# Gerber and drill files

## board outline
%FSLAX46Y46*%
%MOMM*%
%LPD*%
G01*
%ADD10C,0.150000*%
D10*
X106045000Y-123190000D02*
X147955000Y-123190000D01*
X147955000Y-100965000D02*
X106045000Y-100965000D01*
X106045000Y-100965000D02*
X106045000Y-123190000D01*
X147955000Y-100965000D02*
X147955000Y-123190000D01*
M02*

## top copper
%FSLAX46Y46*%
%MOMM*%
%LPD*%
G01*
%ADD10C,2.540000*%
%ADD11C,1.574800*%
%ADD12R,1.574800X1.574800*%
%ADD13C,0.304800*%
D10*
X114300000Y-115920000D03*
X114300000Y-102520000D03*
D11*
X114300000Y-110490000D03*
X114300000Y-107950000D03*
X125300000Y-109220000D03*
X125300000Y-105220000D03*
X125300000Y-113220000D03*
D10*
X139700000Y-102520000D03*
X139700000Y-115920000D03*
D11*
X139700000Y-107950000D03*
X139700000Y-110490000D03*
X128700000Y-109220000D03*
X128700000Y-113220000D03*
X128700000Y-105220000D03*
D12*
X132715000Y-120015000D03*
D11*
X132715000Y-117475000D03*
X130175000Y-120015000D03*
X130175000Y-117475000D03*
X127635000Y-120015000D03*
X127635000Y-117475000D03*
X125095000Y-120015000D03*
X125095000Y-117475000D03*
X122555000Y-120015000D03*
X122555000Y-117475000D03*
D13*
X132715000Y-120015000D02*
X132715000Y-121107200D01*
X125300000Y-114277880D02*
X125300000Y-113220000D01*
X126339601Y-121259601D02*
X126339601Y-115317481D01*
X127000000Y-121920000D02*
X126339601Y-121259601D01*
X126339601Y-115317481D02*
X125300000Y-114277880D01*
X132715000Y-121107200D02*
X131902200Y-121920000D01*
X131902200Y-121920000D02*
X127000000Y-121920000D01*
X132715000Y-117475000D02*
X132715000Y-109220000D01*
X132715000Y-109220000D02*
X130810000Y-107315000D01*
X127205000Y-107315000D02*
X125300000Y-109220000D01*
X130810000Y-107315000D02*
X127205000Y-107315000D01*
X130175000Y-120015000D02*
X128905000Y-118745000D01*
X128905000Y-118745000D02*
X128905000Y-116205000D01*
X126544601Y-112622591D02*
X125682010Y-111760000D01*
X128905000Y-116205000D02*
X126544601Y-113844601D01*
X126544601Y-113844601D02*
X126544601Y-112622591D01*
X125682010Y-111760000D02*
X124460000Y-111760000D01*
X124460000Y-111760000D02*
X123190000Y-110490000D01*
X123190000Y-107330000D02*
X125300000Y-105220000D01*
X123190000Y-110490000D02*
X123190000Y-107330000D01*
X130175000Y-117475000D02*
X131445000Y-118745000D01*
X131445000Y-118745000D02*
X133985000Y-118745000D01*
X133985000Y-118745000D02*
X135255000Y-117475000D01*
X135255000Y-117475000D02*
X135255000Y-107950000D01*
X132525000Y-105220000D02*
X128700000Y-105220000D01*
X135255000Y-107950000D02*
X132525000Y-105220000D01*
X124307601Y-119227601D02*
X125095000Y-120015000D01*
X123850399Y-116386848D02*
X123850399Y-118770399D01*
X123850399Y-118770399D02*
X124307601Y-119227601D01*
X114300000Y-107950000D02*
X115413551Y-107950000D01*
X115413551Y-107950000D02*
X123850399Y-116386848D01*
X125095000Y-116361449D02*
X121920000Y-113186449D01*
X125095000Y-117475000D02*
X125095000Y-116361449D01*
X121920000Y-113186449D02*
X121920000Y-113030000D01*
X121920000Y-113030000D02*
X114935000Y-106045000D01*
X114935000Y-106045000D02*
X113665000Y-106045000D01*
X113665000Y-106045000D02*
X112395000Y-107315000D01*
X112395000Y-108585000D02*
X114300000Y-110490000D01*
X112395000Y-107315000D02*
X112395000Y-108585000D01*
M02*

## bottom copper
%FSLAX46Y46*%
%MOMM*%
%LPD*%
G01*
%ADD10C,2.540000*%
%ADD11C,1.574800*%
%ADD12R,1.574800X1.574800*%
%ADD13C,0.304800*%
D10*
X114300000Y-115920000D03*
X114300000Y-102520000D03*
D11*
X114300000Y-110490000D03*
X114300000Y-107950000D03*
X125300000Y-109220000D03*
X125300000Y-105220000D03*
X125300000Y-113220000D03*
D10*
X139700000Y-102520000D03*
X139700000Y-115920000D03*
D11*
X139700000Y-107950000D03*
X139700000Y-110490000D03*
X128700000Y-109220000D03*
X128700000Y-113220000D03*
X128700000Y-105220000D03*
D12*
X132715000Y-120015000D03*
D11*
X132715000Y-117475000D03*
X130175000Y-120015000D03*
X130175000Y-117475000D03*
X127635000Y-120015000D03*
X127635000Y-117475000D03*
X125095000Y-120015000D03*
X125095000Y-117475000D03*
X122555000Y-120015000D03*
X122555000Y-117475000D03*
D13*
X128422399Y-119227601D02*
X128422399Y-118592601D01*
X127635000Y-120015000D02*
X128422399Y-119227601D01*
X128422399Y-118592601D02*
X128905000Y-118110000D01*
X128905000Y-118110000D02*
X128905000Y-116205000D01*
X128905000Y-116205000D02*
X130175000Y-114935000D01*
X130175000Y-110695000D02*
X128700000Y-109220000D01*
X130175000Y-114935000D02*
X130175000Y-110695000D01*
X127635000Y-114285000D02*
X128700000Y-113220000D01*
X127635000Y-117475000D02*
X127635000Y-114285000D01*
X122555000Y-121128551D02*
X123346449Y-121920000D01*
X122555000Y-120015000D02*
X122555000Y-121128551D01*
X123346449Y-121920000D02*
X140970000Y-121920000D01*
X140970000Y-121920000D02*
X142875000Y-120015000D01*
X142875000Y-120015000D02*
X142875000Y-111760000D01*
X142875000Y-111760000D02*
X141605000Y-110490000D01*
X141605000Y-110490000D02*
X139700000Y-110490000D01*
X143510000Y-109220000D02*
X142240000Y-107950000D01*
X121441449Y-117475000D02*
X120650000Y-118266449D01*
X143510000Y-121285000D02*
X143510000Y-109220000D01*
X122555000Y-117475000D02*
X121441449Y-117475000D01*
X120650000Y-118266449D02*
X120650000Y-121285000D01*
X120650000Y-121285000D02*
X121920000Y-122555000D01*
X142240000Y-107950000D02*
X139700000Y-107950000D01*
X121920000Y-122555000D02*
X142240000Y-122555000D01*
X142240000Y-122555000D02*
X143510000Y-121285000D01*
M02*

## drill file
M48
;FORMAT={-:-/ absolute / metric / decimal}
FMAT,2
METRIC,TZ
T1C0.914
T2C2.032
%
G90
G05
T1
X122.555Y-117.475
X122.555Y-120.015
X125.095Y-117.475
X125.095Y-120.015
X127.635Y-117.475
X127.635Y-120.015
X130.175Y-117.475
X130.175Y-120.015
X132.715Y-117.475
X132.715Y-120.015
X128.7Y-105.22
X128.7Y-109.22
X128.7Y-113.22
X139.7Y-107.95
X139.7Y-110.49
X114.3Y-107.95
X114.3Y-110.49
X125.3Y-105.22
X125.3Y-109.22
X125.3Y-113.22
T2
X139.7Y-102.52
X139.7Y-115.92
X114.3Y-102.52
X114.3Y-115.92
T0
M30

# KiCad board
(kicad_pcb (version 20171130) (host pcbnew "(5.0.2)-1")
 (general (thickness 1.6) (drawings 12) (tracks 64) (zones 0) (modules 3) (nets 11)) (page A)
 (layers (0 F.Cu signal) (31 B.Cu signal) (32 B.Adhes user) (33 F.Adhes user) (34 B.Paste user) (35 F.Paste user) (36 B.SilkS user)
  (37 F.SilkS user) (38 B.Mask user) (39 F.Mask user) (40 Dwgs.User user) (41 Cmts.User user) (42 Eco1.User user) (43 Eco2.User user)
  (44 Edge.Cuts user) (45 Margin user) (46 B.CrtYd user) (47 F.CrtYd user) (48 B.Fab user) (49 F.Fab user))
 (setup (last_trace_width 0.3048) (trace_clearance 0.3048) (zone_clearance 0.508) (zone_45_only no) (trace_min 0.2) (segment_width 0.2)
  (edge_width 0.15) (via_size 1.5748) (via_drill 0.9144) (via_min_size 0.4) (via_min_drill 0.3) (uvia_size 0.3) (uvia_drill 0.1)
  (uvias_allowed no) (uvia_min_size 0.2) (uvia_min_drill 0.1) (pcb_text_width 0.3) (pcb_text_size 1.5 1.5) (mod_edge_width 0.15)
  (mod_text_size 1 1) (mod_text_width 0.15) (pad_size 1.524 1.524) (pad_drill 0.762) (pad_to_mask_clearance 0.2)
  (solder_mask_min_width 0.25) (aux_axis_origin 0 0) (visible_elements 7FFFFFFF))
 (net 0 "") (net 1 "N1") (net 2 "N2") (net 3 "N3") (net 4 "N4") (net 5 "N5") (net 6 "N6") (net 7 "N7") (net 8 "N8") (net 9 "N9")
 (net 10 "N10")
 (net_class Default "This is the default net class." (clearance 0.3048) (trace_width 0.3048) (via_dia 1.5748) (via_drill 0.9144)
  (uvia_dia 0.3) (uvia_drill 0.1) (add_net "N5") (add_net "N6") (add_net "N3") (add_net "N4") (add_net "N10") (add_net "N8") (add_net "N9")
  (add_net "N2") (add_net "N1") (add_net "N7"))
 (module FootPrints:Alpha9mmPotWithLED (layer F.Cu) (at 114.3 109.22 90)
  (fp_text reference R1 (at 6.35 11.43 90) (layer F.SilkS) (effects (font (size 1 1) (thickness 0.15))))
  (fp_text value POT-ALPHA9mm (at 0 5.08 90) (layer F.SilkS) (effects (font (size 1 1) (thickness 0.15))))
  (pad "" thru_hole circle (at -6.7 0 90) (size 2.54 2.54) (drill 2.032) (layers *.Cu *.Mask F.SilkS))
  (pad "" thru_hole circle (at 6.7 0 90) (size 2.54 2.54) (drill 2.032) (layers *.Cu *.Mask F.SilkS))
  (pad 4 thru_hole circle (at -1.27 0 90) (size 1.5748 1.5748) (drill 0.9144) (layers *.Cu *.Mask F.SilkS) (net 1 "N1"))
  (pad 5 thru_hole circle (at 1.27 0 90) (size 1.5748 1.5748) (drill 0.9144) (layers *.Cu *.Mask F.SilkS) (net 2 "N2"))
  (pad 2 thru_hole circle (at 0 11 90) (size 1.5748 1.5748) (drill 0.9144) (layers *.Cu *.Mask F.SilkS) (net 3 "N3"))
  (pad 3 thru_hole circle (at 4 11 90) (size 1.5748 1.5748) (drill 0.9144) (layers *.Cu *.Mask F.SilkS) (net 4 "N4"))
  (pad 1 thru_hole circle (at -4 11 90) (size 1.5748 1.5748) (drill 0.9144) (layers *.Cu *.Mask F.SilkS) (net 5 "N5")))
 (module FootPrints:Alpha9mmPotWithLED (layer F.Cu) (at 139.7 109.22 270)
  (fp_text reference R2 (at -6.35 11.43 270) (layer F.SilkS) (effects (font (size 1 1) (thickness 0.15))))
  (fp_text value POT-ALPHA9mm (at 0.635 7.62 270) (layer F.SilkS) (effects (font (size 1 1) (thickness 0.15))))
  (pad "" thru_hole circle (at -6.7 0 270) (size 2.54 2.54) (drill 2.032) (layers *.Cu *.Mask F.SilkS))
  (pad "" thru_hole circle (at 6.7 0 270) (size 2.54 2.54) (drill 2.032) (layers *.Cu *.Mask F.SilkS))
  (pad 4 thru_hole circle (at -1.27 0 270) (size 1.5748 1.5748) (drill 0.9144) (layers *.Cu *.Mask F.SilkS) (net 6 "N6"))
  (pad 5 thru_hole circle (at 1.27 0 270) (size 1.5748 1.5748) (drill 0.9144) (layers *.Cu *.Mask F.SilkS) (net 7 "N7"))
  (pad 2 thru_hole circle (at 0 11 270) (size 1.5748 1.5748) (drill 0.9144) (layers *.Cu *.Mask F.SilkS) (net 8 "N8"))
  (pad 3 thru_hole circle (at 4 11 270) (size 1.5748 1.5748) (drill 0.9144) (layers *.Cu *.Mask F.SilkS) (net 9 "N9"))
  (pad 1 thru_hole circle (at -4 11 270) (size 1.5748 1.5748) (drill 0.9144) (layers *.Cu *.Mask F.SilkS) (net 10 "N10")))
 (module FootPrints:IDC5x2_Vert (layer B.Cu) (at 127.635 118.745)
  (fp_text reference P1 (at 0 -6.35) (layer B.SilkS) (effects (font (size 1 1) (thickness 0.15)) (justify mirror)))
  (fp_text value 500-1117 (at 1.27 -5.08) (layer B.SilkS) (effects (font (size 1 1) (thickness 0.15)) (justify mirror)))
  (pad 1 thru_hole rect (at 5.08 1.27) (size 1.5748 1.5748) (drill 0.9144) (layers *.Cu *.Mask B.SilkS) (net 5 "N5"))
  (pad 2 thru_hole circle (at 5.08 -1.27) (size 1.5748 1.5748) (drill 0.9144) (layers *.Cu *.Mask B.SilkS) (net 3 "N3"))
  (pad 3 thru_hole circle (at 2.54 1.27) (size 1.5748 1.5748) (drill 0.9144) (layers *.Cu *.Mask B.SilkS) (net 4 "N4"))
  (pad 4 thru_hole circle (at 2.54 -1.27) (size 1.5748 1.5748) (drill 0.9144) (layers *.Cu *.Mask B.SilkS) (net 10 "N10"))
  (pad 5 thru_hole circle (at 0 1.27) (size 1.5748 1.5748) (drill 0.9144) (layers *.Cu *.Mask B.SilkS) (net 8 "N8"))
  (pad 6 thru_hole circle (at 0 -1.27) (size 1.5748 1.5748) (drill 0.9144) (layers *.Cu *.Mask B.SilkS) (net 9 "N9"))
  (pad 7 thru_hole circle (at -2.54 1.27) (size 1.5748 1.5748) (drill 0.9144) (layers *.Cu *.Mask B.SilkS) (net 2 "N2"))
  (pad 8 thru_hole circle (at -2.54 -1.27) (size 1.5748 1.5748) (drill 0.9144) (layers *.Cu *.Mask B.SilkS) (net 1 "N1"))
  (pad 9 thru_hole circle (at -5.08 1.27) (size 1.5748 1.5748) (drill 0.9144) (layers *.Cu *.Mask B.SilkS) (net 7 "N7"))
  (pad 10 thru_hole circle (at -5.08 -1.27) (size 1.5748 1.5748) (drill 0.9144) (layers *.Cu *.Mask B.SilkS) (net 6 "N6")))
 (gr_line (start 106.045 123.19) (end 147.955 123.19) (layer Edge.Cuts) (width 0.15))
 (gr_line (start 147.955 100.965) (end 106.045 100.965) (layer Edge.Cuts) (width 0.15))
 (gr_line (start 106.045 100.965) (end 106.045 123.19) (layer Edge.Cuts) (width 0.15))
 (gr_line (start 147.955 100.965) (end 147.955 123.19) (layer Edge.Cuts) (width 0.15))
 (segment (start 132.715 120.015) (end 132.715 121.1072) (width 0.3048) (layer F.Cu) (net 5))
 (segment (start 125.3 114.27788) (end 125.3 113.22) (width 0.3048) (layer F.Cu) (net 5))
 (segment (start 126.339601 121.259601) (end 126.339601 115.317481) (width 0.3048) (layer F.Cu) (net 5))
 (segment (start 127 121.92) (end 126.339601 121.259601) (width 0.3048) (layer F.Cu) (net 5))
 (segment (start 126.339601 115.317481) (end 125.3 114.27788) (width 0.3048) (layer F.Cu) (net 5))
 (segment (start 132.715 121.1072) (end 131.9022 121.92) (width 0.3048) (layer F.Cu) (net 5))
 (segment (start 131.9022 121.92) (end 127 121.92) (width 0.3048) (layer F.Cu) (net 5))
 (segment (start 132.715 117.475) (end 132.715 109.22) (width 0.3048) (layer F.Cu) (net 3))
 (segment (start 132.715 109.22) (end 130.81 107.315) (width 0.3048) (layer F.Cu) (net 3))
 (segment (start 127.205 107.315) (end 125.3 109.22) (width 0.3048) (layer F.Cu) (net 3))
 (segment (start 130.81 107.315) (end 127.205 107.315) (width 0.3048) (layer F.Cu) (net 3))
 (segment (start 130.175 120.015) (end 128.905 118.745) (width 0.3048) (layer F.Cu) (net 4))
 (segment (start 128.905 118.745) (end 128.905 116.205) (width 0.3048) (layer F.Cu) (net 4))
 (segment (start 126.544601 112.622591) (end 125.68201 111.76) (width 0.3048) (layer F.Cu) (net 4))
 (segment (start 128.905 116.205) (end 126.544601 113.844601) (width 0.3048) (layer F.Cu) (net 4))
 (segment (start 126.544601 113.844601) (end 126.544601 112.622591) (width 0.3048) (layer F.Cu) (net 4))
 (segment (start 125.68201 111.76) (end 124.46 111.76) (width 0.3048) (layer F.Cu) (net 4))
 (segment (start 124.46 111.76) (end 123.19 110.49) (width 0.3048) (layer F.Cu) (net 4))
 (segment (start 123.19 107.33) (end 125.3 105.22) (width 0.3048) (layer F.Cu) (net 4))
 (segment (start 123.19 110.49) (end 123.19 107.33) (width 0.3048) (layer F.Cu) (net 4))
 (segment (start 130.175 117.475) (end 131.445 118.745) (width 0.3048) (layer F.Cu) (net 10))
 (segment (start 131.445 118.745) (end 133.985 118.745) (width 0.3048) (layer F.Cu) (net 10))
 (segment (start 133.985 118.745) (end 135.255 117.475) (width 0.3048) (layer F.Cu) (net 10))
 (segment (start 135.255 117.475) (end 135.255 107.95) (width 0.3048) (layer F.Cu) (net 10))
 (segment (start 132.525 105.22) (end 128.7 105.22) (width 0.3048) (layer F.Cu) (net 10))
 (segment (start 135.255 107.95) (end 132.525 105.22) (width 0.3048) (layer F.Cu) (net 10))
 (segment (start 128.422399 119.227601) (end 128.422399 118.592601) (width 0.3048) (layer B.Cu) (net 8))
 (segment (start 127.635 120.015) (end 128.422399 119.227601) (width 0.3048) (layer B.Cu) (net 8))
 (segment (start 128.422399 118.592601) (end 128.905 118.11) (width 0.3048) (layer B.Cu) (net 8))
 (segment (start 128.905 118.11) (end 128.905 116.205) (width 0.3048) (layer B.Cu) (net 8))
 (segment (start 128.905 116.205) (end 130.175 114.935) (width 0.3048) (layer B.Cu) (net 8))
 (segment (start 130.175 110.695) (end 128.7 109.22) (width 0.3048) (layer B.Cu) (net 8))
 (segment (start 130.175 114.935) (end 130.175 110.695) (width 0.3048) (layer B.Cu) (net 8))
 (segment (start 127.635 114.285) (end 128.7 113.22) (width 0.3048) (layer B.Cu) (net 9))
 (segment (start 127.635 117.475) (end 127.635 114.285) (width 0.3048) (layer B.Cu) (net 9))
 (segment (start 124.307601 119.227601) (end 125.095 120.015) (width 0.3048) (layer F.Cu) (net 2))
 (segment (start 123.850399 116.386848) (end 123.850399 118.770399) (width 0.3048) (layer F.Cu) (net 2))
 (segment (start 123.850399 118.770399) (end 124.307601 119.227601) (width 0.3048) (layer F.Cu) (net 2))
 (segment (start 114.3 107.95) (end 115.413551 107.95) (width 0.3048) (layer F.Cu) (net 2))
 (segment (start 115.413551 107.95) (end 123.850399 116.386848) (width 0.3048) (layer F.Cu) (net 2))
 (segment (start 125.095 116.361449) (end 121.92 113.186449) (width 0.3048) (layer F.Cu) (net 1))
 (segment (start 125.095 117.475) (end 125.095 116.361449) (width 0.3048) (layer F.Cu) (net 1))
 (segment (start 121.92 113.186449) (end 121.92 113.03) (width 0.3048) (layer F.Cu) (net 1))
 (segment (start 121.92 113.03) (end 114.935 106.045) (width 0.3048) (layer F.Cu) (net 1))
 (segment (start 114.935 106.045) (end 113.665 106.045) (width 0.3048) (layer F.Cu) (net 1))
 (segment (start 113.665 106.045) (end 112.395 107.315) (width 0.3048) (layer F.Cu) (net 1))
 (segment (start 112.395 108.585) (end 114.3 110.49) (width 0.3048) (layer F.Cu) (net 1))
 (segment (start 112.395 107.315) (end 112.395 108.585) (width 0.3048) (layer F.Cu) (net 1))
 (segment (start 122.555 121.128551) (end 123.346449 121.92) (width 0.3048) (layer B.Cu) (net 7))
 (segment (start 122.555 120.015) (end 122.555 121.128551) (width 0.3048) (layer B.Cu) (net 7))
 (segment (start 123.346449 121.92) (end 140.97 121.92) (width 0.3048) (layer B.Cu) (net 7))
 (segment (start 140.97 121.92) (end 142.875 120.015) (width 0.3048) (layer B.Cu) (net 7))
 (segment (start 142.875 120.015) (end 142.875 111.76) (width 0.3048) (layer B.Cu) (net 7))
 (segment (start 142.875 111.76) (end 141.605 110.49) (width 0.3048) (layer B.Cu) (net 7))
 (segment (start 141.605 110.49) (end 139.7 110.49) (width 0.3048) (layer B.Cu) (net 7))
 (segment (start 143.51 109.22) (end 142.24 107.95) (width 0.3048) (layer B.Cu) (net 6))
 (segment (start 121.441449 117.475) (end 120.65 118.266449) (width 0.3048) (layer B.Cu) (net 6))
 (segment (start 143.51 121.285) (end 143.51 109.22) (width 0.3048) (layer B.Cu) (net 6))
 (segment (start 122.555 117.475) (end 121.441449 117.475) (width 0.3048) (layer B.Cu) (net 6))
 (segment (start 120.65 118.266449) (end 120.65 121.285) (width 0.3048) (layer B.Cu) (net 6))
 (segment (start 120.65 121.285) (end 121.92 122.555) (width 0.3048) (layer B.Cu) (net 6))
 (segment (start 142.24 107.95) (end 139.7 107.95) (width 0.3048) (layer B.Cu) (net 6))
 (segment (start 121.92 122.555) (end 142.24 122.555) (width 0.3048) (layer B.Cu) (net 6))
 (segment (start 142.24 122.555) (end 143.51 121.285) (width 0.3048) (layer B.Cu) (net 6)))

